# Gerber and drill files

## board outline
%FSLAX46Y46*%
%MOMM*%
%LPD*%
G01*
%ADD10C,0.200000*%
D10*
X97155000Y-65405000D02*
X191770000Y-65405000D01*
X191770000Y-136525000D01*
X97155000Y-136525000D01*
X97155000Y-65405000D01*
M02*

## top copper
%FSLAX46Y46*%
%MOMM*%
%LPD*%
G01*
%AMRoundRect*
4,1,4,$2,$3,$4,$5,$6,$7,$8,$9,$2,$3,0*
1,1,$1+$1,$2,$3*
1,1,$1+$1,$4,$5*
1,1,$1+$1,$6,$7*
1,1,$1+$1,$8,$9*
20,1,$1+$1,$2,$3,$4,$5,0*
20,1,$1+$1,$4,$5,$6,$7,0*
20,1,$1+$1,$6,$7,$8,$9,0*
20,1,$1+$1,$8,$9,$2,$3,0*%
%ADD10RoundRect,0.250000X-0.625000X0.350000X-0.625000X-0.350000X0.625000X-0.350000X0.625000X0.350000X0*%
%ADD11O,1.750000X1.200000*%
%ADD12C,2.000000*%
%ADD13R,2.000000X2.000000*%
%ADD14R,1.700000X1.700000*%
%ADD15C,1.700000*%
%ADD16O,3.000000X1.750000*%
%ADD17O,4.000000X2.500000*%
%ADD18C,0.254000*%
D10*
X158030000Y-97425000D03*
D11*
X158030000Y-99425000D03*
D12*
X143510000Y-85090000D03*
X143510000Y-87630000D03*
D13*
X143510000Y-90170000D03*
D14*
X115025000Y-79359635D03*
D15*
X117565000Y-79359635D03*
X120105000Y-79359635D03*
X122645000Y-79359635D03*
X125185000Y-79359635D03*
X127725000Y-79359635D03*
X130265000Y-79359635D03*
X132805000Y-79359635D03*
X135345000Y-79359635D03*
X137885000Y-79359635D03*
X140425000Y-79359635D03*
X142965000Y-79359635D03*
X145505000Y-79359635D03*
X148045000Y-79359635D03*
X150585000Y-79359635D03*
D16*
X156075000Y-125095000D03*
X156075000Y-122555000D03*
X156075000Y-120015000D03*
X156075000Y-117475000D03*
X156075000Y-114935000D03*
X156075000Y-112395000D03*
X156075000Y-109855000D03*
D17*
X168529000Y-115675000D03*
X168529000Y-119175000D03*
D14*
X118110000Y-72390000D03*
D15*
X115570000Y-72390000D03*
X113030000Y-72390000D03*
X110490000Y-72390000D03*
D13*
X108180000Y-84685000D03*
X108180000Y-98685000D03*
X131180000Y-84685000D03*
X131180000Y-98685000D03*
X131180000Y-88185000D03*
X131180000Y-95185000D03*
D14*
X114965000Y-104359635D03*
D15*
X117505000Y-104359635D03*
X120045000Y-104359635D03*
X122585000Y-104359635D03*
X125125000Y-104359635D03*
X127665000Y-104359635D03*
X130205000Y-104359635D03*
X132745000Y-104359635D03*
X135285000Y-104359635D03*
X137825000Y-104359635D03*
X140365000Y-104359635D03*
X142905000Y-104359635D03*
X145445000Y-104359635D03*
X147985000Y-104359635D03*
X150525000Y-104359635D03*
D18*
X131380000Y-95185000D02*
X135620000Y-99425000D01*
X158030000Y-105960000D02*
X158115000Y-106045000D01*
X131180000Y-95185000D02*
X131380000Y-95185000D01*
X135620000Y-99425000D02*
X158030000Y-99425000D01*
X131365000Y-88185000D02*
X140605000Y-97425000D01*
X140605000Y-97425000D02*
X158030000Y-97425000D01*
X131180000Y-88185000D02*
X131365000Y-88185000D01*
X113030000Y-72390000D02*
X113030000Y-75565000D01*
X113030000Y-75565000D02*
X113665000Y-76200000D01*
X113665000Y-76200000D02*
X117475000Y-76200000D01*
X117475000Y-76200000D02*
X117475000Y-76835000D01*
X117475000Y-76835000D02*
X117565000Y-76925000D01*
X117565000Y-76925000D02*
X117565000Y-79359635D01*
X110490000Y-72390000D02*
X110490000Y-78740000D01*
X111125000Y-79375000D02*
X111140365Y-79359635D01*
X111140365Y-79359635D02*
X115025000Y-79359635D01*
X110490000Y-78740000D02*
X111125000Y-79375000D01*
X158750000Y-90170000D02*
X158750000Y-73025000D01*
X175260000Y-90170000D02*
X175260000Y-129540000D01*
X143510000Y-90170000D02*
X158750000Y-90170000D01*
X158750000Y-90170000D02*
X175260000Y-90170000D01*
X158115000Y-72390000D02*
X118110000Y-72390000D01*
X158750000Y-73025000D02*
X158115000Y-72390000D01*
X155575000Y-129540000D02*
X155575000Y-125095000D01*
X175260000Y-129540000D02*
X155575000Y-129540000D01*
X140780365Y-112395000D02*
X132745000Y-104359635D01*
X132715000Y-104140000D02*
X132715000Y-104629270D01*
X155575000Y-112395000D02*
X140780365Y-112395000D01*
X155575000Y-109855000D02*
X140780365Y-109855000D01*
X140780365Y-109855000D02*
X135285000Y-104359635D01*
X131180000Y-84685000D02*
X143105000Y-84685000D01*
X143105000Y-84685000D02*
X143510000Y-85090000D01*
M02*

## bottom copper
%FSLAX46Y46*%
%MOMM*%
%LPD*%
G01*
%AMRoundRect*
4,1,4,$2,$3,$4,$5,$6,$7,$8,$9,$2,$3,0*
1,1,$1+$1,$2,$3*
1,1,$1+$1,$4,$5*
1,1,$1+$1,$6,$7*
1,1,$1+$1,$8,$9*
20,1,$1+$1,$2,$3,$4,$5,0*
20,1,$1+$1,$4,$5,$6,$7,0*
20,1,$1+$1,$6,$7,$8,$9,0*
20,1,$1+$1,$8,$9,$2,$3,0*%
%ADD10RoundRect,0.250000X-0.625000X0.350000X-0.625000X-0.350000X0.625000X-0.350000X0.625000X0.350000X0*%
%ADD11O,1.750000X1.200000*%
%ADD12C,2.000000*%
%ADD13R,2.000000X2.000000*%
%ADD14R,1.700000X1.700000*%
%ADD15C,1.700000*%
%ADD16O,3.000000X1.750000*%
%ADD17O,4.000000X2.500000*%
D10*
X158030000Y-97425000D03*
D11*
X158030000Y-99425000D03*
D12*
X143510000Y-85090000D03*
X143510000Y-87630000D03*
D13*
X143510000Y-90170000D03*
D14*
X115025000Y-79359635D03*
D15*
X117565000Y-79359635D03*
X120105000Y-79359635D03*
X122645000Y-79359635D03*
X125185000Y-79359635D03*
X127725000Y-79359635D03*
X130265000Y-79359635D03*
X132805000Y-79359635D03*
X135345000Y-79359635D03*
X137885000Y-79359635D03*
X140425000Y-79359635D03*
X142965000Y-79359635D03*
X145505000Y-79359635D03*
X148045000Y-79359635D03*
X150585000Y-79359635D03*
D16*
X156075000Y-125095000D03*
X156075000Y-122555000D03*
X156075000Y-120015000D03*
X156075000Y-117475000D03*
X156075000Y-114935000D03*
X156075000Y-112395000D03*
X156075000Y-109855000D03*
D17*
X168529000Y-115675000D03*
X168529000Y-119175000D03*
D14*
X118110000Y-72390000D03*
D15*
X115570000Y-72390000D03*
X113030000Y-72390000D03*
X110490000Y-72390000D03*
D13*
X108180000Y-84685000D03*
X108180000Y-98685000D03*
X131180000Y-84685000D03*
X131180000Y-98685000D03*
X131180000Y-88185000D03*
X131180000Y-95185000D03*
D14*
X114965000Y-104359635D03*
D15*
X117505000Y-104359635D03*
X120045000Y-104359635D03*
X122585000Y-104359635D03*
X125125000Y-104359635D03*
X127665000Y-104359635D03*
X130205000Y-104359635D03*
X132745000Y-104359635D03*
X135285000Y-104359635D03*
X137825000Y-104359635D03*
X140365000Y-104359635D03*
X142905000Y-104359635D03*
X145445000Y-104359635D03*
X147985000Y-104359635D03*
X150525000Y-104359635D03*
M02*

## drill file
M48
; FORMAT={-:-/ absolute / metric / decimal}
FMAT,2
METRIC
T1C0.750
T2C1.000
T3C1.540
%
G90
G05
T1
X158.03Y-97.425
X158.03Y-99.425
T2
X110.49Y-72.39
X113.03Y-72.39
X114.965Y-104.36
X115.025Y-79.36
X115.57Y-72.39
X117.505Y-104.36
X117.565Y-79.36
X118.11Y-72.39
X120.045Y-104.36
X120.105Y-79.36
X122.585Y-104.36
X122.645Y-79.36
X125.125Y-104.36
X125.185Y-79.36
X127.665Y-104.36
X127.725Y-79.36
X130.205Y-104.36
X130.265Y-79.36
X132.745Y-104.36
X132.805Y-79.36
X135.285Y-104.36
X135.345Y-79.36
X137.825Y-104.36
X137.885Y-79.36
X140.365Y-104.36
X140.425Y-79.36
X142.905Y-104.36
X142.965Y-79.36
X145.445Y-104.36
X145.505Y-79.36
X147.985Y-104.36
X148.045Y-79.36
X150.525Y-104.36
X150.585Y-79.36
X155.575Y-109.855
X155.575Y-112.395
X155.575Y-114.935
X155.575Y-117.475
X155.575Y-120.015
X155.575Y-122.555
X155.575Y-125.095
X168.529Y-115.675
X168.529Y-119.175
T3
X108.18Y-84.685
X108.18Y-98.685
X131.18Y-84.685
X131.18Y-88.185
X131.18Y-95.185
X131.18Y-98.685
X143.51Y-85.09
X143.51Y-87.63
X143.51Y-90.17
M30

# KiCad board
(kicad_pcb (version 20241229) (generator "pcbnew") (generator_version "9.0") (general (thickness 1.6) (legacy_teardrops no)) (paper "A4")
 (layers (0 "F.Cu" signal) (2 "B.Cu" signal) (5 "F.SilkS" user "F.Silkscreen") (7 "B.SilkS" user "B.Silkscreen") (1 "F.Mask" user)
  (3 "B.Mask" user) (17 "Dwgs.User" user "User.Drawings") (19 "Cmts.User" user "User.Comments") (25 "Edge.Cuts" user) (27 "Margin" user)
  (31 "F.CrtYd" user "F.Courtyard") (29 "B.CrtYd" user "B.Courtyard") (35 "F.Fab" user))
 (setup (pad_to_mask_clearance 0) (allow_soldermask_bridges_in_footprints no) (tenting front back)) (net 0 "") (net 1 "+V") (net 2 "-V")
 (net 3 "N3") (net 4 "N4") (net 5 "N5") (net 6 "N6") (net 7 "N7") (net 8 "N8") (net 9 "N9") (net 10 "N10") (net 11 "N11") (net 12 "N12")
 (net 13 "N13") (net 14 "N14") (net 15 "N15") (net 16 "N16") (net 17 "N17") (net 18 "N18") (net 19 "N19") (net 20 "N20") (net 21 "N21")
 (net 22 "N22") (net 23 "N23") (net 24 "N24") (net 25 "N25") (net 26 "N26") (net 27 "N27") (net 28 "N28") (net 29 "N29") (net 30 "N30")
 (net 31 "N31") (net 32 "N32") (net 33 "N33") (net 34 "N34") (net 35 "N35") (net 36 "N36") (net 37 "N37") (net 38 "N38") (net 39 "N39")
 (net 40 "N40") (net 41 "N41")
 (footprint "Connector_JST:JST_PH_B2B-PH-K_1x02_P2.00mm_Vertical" (layer "F.Cu") (at 158.03 97.425 -90)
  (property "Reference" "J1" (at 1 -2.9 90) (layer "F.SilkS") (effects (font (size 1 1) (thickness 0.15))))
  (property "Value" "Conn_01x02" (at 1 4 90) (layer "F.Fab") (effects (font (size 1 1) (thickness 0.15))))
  (pad "1" thru_hole roundrect (at 0 0 270) (size 1.2 1.75) (drill 0.75) (layers "*.Cu" "*.Mask") (remove_unused_layers no)
   (roundrect_rratio 0.208333) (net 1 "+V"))
  (pad "2" thru_hole oval (at 2 0 270) (size 1.2 1.75) (drill 0.75) (layers "*.Cu" "*.Mask") (remove_unused_layers no) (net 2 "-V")))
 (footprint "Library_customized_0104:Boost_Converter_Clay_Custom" (layer "F.Cu") (at 147.26 87.38)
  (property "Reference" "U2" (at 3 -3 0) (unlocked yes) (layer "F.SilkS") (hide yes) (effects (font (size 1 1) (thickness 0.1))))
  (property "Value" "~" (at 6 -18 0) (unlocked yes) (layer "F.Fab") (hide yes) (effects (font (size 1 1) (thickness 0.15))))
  (pad "1" thru_hole circle (at -3.75 -2.29) (size 2 2) (drill 1.54) (layers "*.Cu" "*.Mask") (remove_unused_layers no) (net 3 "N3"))
  (pad "2" thru_hole circle (at -3.75 0.25) (size 2 2) (drill 1.54) (layers "*.Cu" "*.Mask") (remove_unused_layers no) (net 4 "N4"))
  (pad "3" thru_hole rect (at -3.75 2.79) (size 2 2) (drill 1.54) (layers "*.Cu" "*.Mask") (remove_unused_layers no) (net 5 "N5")))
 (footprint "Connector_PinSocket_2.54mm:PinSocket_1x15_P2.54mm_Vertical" (layer "F.Cu") (at 115.025 79.359635 90)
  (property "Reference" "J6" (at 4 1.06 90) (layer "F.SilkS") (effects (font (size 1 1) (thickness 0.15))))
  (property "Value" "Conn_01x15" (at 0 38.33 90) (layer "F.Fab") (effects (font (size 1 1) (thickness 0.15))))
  (pad "1" thru_hole rect (at 0 0 90) (size 1.7 1.7) (drill 1) (layers "*.Cu" "*.Mask") (remove_unused_layers no) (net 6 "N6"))
  (pad "2" thru_hole circle (at 0 2.54 90) (size 1.7 1.7) (drill 1) (layers "*.Cu" "*.Mask") (remove_unused_layers no) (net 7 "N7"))
  (pad "3" thru_hole circle (at 0 5.08 90) (size 1.7 1.7) (drill 1) (layers "*.Cu" "*.Mask") (remove_unused_layers no) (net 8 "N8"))
  (pad "4" thru_hole circle (at 0 7.62 90) (size 1.7 1.7) (drill 1) (layers "*.Cu" "*.Mask") (remove_unused_layers no) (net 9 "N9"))
  (pad "5" thru_hole circle (at 0 10.16 90) (size 1.7 1.7) (drill 1) (layers "*.Cu" "*.Mask") (remove_unused_layers no) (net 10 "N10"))
  (pad "6" thru_hole circle (at 0 12.7 90) (size 1.7 1.7) (drill 1) (layers "*.Cu" "*.Mask") (remove_unused_layers no) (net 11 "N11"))
  (pad "7" thru_hole circle (at 0 15.24 90) (size 1.7 1.7) (drill 1) (layers "*.Cu" "*.Mask") (remove_unused_layers no) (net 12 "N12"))
  (pad "8" thru_hole circle (at 0 17.78 90) (size 1.7 1.7) (drill 1) (layers "*.Cu" "*.Mask") (remove_unused_layers no) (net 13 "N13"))
  (pad "9" thru_hole circle (at 0 20.32 90) (size 1.7 1.7) (drill 1) (layers "*.Cu" "*.Mask") (remove_unused_layers no) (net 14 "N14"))
  (pad "10" thru_hole circle (at 0 22.86 90) (size 1.7 1.7) (drill 1) (layers "*.Cu" "*.Mask") (remove_unused_layers no) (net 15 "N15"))
  (pad "11" thru_hole circle (at 0 25.4 90) (size 1.7 1.7) (drill 1) (layers "*.Cu" "*.Mask") (remove_unused_layers no) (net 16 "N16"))
  (pad "12" thru_hole circle (at 0 27.94 90) (size 1.7 1.7) (drill 1) (layers "*.Cu" "*.Mask") (remove_unused_layers no) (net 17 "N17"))
  (pad "13" thru_hole circle (at 0 30.48 90) (size 1.7 1.7) (drill 1) (layers "*.Cu" "*.Mask") (remove_unused_layers no) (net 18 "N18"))
  (pad "14" thru_hole circle (at 0 33.02 90) (size 1.7 1.7) (drill 1) (layers "*.Cu" "*.Mask") (remove_unused_layers no) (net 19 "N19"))
  (pad "15" thru_hole circle (at 0 35.56 90) (size 1.7 1.7) (drill 1) (layers "*.Cu" "*.Mask") (remove_unused_layers no) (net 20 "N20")))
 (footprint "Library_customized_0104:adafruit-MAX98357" (layer "F.Cu") (at 162.482 117.595 -90)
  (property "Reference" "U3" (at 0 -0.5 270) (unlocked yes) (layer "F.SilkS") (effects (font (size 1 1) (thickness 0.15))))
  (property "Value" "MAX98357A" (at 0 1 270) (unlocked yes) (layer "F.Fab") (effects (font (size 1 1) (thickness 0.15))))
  (pad "1" thru_hole oval (at 7.5 6.907 180) (size 3 1.75) (drill 1 (offset -0.5 0)) (layers "*.Cu" "*.Mask") (remove_unused_layers no)
   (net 5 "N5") (solder_mask_margin 0.0508))
  (pad "2" thru_hole oval (at 4.96 6.907 180) (size 3 1.75) (drill 1 (offset -0.5 0)) (layers "*.Cu" "*.Mask") (remove_unused_layers no)
   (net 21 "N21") (solder_mask_margin 0.0508))
  (pad "3" thru_hole oval (at 2.42 6.907 180) (size 3 1.75) (drill 1 (offset -0.5 0)) (layers "*.Cu" "*.Mask") (remove_unused_layers no)
   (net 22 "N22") (solder_mask_margin 0.0508))
  (pad "4" thru_hole oval (at -0.12 6.907 180) (size 3 1.75) (drill 1 (offset -0.5 0)) (layers "*.Cu" "*.Mask") (remove_unused_layers no)
   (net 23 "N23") (solder_mask_margin 0.0508))
  (pad "5" thru_hole oval (at -2.66 6.907 180) (size 3 1.75) (drill 1 (offset -0.5 0)) (layers "*.Cu" "*.Mask") (remove_unused_layers no)
   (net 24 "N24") (solder_mask_margin 0.0508))
  (pad "6" thru_hole oval (at -5.2 6.907 180) (size 3 1.75) (drill 1 (offset -0.5 0)) (layers "*.Cu" "*.Mask") (remove_unused_layers no)
   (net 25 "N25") (solder_mask_margin 0.0508))
  (pad "7" thru_hole oval (at -7.74 6.907 180) (size 3 1.75) (drill 1 (offset -0.5 0)) (layers "*.Cu" "*.Mask") (remove_unused_layers no)
   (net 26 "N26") (solder_mask_margin 0.0508))
  (pad "8" thru_hole oval (at -1.92 -6.047 90) (size 2.5 4) (drill 1) (layers "*.Cu" "*.Mask") (remove_unused_layers no) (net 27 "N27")
   (solder_mask_margin 0.0508))
  (pad "9" thru_hole oval (at 1.58 -6.047 90) (size 2.5 4) (drill 1) (layers "*.Cu" "*.Mask") (remove_unused_layers no) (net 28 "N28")
   (solder_mask_margin 0.0508)))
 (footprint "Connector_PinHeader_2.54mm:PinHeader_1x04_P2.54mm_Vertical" (layer "F.Cu") (at 118.11 72.39 -90)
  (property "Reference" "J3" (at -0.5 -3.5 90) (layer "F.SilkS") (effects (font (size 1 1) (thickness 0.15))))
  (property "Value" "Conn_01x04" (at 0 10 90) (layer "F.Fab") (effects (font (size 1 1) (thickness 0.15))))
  (pad "1" thru_hole rect (at 0 0 270) (size 1.7 1.7) (drill 1) (layers "*.Cu" "*.Mask") (remove_unused_layers no) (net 5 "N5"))
  (pad "2" thru_hole circle (at 0 2.54 270) (size 1.7 1.7) (drill 1) (layers "*.Cu" "*.Mask") (remove_unused_layers no) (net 21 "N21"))
  (pad "3" thru_hole circle (at 0 5.08 270) (size 1.7 1.7) (drill 1) (layers "*.Cu" "*.Mask") (remove_unused_layers no) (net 7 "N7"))
  (pad "4" thru_hole circle (at 0 7.62 270) (size 1.7 1.7) (drill 1) (layers "*.Cu" "*.Mask") (remove_unused_layers no) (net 6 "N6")))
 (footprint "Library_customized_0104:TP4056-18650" (layer "F.Cu") (at 106.68 83.185)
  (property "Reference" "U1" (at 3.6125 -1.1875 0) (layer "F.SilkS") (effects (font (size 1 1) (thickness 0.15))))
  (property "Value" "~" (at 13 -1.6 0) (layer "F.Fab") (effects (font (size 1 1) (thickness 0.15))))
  (pad "1" thru_hole rect (at 1.5 1.5) (size 2 2) (drill 1.54) (layers "*.Cu" "*.Mask") (remove_unused_layers no) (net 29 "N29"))
  (pad "2" thru_hole rect (at 1.5 15.5) (size 2 2) (drill 1.54) (layers "*.Cu" "*.Mask") (remove_unused_layers no) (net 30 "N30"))
  (pad "3" thru_hole rect (at 24.5 1.5) (size 2 2) (drill 1.54) (layers "*.Cu" "*.Mask") (remove_unused_layers no) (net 3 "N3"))
  (pad "4" thru_hole rect (at 24.5 15.5) (size 2 2) (drill 1.54) (layers "*.Cu" "*.Mask") (remove_unused_layers no) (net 4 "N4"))
  (pad "5" thru_hole rect (at 24.5 5) (size 2 2) (drill 1.54) (layers "*.Cu" "*.Mask") (remove_unused_layers no) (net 1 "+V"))
  (pad "6" thru_hole rect (at 24.5 12) (size 2 2) (drill 1.54) (layers "*.Cu" "*.Mask") (remove_unused_layers no) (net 2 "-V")))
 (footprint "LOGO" (layer "F.Cu") (at 148.105 37.18)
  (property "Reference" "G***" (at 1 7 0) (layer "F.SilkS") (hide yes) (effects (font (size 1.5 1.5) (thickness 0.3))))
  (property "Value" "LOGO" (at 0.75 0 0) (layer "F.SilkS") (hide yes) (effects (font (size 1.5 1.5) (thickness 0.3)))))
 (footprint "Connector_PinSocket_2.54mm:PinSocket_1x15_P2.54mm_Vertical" (layer "F.Cu") (at 114.965 104.359635 90)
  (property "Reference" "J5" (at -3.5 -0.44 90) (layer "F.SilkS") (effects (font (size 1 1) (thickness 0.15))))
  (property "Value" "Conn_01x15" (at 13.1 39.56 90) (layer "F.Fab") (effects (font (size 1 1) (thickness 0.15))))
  (pad "1" thru_hole rect (at 0 0 90) (size 1.7 1.7) (drill 1) (layers "*.Cu" "*.Mask") (remove_unused_layers no) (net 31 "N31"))
  (pad "2" thru_hole circle (at 0 2.54 90) (size 1.7 1.7) (drill 1) (layers "*.Cu" "*.Mask") (remove_unused_layers no) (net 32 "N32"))
  (pad "3" thru_hole circle (at 0 5.08 90) (size 1.7 1.7) (drill 1) (layers "*.Cu" "*.Mask") (remove_unused_layers no) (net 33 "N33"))
  (pad "4" thru_hole circle (at 0 7.62 90) (size 1.7 1.7) (drill 1) (layers "*.Cu" "*.Mask") (remove_unused_layers no) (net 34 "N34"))
  (pad "5" thru_hole circle (at 0 10.16 90) (size 1.7 1.7) (drill 1) (layers "*.Cu" "*.Mask") (remove_unused_layers no) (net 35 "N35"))
  (pad "6" thru_hole circle (at 0 12.7 90) (size 1.7 1.7) (drill 1) (layers "*.Cu" "*.Mask") (remove_unused_layers no) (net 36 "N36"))
  (pad "7" thru_hole circle (at 0 15.24 90) (size 1.7 1.7) (drill 1) (layers "*.Cu" "*.Mask") (remove_unused_layers no) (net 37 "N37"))
  (pad "8" thru_hole circle (at 0 17.78 90) (size 1.7 1.7) (drill 1) (layers "*.Cu" "*.Mask") (remove_unused_layers no) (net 25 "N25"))
  (pad "9" thru_hole circle (at 0 20.32 90) (size 1.7 1.7) (drill 1) (layers "*.Cu" "*.Mask") (remove_unused_layers no) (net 26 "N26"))
  (pad "10" thru_hole circle (at 0 22.86 90) (size 1.7 1.7) (drill 1) (layers "*.Cu" "*.Mask") (remove_unused_layers no) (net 24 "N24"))
  (pad "11" thru_hole circle (at 0 25.4 90) (size 1.7 1.7) (drill 1) (layers "*.Cu" "*.Mask") (remove_unused_layers no) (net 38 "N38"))
  (pad "12" thru_hole circle (at 0 27.94 90) (size 1.7 1.7) (drill 1) (layers "*.Cu" "*.Mask") (remove_unused_layers no) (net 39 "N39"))
  (pad "13" thru_hole circle (at 0 30.48 90) (size 1.7 1.7) (drill 1) (layers "*.Cu" "*.Mask") (remove_unused_layers no) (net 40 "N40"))
  (pad "14" thru_hole circle (at 0 33.02 90) (size 1.7 1.7) (drill 1) (layers "*.Cu" "*.Mask") (remove_unused_layers no) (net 21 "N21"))
  (pad "15" thru_hole circle (at 0 35.56 90) (size 1.7 1.7) (drill 1) (layers "*.Cu" "*.Mask") (remove_unused_layers no) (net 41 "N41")))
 (gr_rect (start 97.155 65.405) (end 191.77 136.525) (stroke (width 0.2) (type solid)) (fill no) (layer "Edge.Cuts"))
 (segment (start 131.38 95.185) (end 135.62 99.425) (width 0.254) (layer "F.Cu") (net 2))
 (segment (start 158.03 105.96) (end 158.115 106.045) (width 0.254) (layer "F.Cu") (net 2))
 (segment (start 131.18 95.185) (end 131.38 95.185) (width 0.254) (layer "F.Cu") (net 2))
 (segment (start 135.62 99.425) (end 158.03 99.425) (width 0.254) (layer "F.Cu") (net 2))
 (segment (start 131.365 88.185) (end 140.605 97.425) (width 0.254) (layer "F.Cu") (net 1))
 (segment (start 140.605 97.425) (end 158.03 97.425) (width 0.254) (layer "F.Cu") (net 1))
 (segment (start 131.18 88.185) (end 131.365 88.185) (width 0.254) (layer "F.Cu") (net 1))
 (segment (start 113.03 72.39) (end 113.03 75.565) (width 0.254) (layer "F.Cu") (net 7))
 (segment (start 113.03 75.565) (end 113.665 76.2) (width 0.254) (layer "F.Cu") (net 7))
 (segment (start 113.665 76.2) (end 117.475 76.2) (width 0.254) (layer "F.Cu") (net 7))
 (segment (start 117.475 76.2) (end 117.475 76.835) (width 0.254) (layer "F.Cu") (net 7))
 (segment (start 117.475 76.835) (end 117.565 76.925) (width 0.254) (layer "F.Cu") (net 7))
 (segment (start 117.565 76.925) (end 117.565 79.359635) (width 0.254) (layer "F.Cu") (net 7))
 (segment (start 110.49 72.39) (end 110.49 78.74) (width 0.254) (layer "F.Cu") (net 6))
 (segment (start 111.125 79.375) (end 111.140365 79.359635) (width 0.254) (layer "F.Cu") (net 6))
 (segment (start 111.140365 79.359635) (end 115.025 79.359635) (width 0.254) (layer "F.Cu") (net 6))
 (segment (start 110.49 78.74) (end 111.125 79.375) (width 0.254) (layer "F.Cu") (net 6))
 (segment (start 158.75 90.17) (end 158.75 73.025) (width 0.254) (layer "F.Cu") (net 5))
 (segment (start 175.26 90.17) (end 175.26 129.54) (width 0.254) (layer "F.Cu") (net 5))
 (segment (start 143.51 90.17) (end 158.75 90.17) (width 0.254) (layer "F.Cu") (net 5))
 (segment (start 158.75 90.17) (end 175.26 90.17) (width 0.254) (layer "F.Cu") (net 5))
 (segment (start 158.115 72.39) (end 118.11 72.39) (width 0.254) (layer "F.Cu") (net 5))
 (segment (start 158.75 73.025) (end 158.115 72.39) (width 0.254) (layer "F.Cu") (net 5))
 (segment (start 155.575 129.54) (end 155.575 125.095) (width 0.254) (layer "F.Cu") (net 5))
 (segment (start 175.26 129.54) (end 155.575 129.54) (width 0.254) (layer "F.Cu") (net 5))
 (segment (start 140.780365 112.395) (end 132.745 104.359635) (width 0.254) (layer "F.Cu") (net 25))
 (segment (start 132.715 104.14) (end 132.715 104.62927) (width 0.254) (layer "F.Cu") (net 25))
 (segment (start 155.575 112.395) (end 140.780365 112.395) (width 0.254) (layer "F.Cu") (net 25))
 (segment (start 155.575 109.855) (end 140.780365 109.855) (width 0.254) (layer "F.Cu") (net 26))
 (segment (start 140.780365 109.855) (end 135.285 104.359635) (width 0.254) (layer "F.Cu") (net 26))
 (segment (start 131.18 84.685) (end 143.105 84.685) (width 0.254) (layer "F.Cu") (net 3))
 (segment (start 143.105 84.685) (end 143.51 85.09) (width 0.254) (layer "F.Cu") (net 3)))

